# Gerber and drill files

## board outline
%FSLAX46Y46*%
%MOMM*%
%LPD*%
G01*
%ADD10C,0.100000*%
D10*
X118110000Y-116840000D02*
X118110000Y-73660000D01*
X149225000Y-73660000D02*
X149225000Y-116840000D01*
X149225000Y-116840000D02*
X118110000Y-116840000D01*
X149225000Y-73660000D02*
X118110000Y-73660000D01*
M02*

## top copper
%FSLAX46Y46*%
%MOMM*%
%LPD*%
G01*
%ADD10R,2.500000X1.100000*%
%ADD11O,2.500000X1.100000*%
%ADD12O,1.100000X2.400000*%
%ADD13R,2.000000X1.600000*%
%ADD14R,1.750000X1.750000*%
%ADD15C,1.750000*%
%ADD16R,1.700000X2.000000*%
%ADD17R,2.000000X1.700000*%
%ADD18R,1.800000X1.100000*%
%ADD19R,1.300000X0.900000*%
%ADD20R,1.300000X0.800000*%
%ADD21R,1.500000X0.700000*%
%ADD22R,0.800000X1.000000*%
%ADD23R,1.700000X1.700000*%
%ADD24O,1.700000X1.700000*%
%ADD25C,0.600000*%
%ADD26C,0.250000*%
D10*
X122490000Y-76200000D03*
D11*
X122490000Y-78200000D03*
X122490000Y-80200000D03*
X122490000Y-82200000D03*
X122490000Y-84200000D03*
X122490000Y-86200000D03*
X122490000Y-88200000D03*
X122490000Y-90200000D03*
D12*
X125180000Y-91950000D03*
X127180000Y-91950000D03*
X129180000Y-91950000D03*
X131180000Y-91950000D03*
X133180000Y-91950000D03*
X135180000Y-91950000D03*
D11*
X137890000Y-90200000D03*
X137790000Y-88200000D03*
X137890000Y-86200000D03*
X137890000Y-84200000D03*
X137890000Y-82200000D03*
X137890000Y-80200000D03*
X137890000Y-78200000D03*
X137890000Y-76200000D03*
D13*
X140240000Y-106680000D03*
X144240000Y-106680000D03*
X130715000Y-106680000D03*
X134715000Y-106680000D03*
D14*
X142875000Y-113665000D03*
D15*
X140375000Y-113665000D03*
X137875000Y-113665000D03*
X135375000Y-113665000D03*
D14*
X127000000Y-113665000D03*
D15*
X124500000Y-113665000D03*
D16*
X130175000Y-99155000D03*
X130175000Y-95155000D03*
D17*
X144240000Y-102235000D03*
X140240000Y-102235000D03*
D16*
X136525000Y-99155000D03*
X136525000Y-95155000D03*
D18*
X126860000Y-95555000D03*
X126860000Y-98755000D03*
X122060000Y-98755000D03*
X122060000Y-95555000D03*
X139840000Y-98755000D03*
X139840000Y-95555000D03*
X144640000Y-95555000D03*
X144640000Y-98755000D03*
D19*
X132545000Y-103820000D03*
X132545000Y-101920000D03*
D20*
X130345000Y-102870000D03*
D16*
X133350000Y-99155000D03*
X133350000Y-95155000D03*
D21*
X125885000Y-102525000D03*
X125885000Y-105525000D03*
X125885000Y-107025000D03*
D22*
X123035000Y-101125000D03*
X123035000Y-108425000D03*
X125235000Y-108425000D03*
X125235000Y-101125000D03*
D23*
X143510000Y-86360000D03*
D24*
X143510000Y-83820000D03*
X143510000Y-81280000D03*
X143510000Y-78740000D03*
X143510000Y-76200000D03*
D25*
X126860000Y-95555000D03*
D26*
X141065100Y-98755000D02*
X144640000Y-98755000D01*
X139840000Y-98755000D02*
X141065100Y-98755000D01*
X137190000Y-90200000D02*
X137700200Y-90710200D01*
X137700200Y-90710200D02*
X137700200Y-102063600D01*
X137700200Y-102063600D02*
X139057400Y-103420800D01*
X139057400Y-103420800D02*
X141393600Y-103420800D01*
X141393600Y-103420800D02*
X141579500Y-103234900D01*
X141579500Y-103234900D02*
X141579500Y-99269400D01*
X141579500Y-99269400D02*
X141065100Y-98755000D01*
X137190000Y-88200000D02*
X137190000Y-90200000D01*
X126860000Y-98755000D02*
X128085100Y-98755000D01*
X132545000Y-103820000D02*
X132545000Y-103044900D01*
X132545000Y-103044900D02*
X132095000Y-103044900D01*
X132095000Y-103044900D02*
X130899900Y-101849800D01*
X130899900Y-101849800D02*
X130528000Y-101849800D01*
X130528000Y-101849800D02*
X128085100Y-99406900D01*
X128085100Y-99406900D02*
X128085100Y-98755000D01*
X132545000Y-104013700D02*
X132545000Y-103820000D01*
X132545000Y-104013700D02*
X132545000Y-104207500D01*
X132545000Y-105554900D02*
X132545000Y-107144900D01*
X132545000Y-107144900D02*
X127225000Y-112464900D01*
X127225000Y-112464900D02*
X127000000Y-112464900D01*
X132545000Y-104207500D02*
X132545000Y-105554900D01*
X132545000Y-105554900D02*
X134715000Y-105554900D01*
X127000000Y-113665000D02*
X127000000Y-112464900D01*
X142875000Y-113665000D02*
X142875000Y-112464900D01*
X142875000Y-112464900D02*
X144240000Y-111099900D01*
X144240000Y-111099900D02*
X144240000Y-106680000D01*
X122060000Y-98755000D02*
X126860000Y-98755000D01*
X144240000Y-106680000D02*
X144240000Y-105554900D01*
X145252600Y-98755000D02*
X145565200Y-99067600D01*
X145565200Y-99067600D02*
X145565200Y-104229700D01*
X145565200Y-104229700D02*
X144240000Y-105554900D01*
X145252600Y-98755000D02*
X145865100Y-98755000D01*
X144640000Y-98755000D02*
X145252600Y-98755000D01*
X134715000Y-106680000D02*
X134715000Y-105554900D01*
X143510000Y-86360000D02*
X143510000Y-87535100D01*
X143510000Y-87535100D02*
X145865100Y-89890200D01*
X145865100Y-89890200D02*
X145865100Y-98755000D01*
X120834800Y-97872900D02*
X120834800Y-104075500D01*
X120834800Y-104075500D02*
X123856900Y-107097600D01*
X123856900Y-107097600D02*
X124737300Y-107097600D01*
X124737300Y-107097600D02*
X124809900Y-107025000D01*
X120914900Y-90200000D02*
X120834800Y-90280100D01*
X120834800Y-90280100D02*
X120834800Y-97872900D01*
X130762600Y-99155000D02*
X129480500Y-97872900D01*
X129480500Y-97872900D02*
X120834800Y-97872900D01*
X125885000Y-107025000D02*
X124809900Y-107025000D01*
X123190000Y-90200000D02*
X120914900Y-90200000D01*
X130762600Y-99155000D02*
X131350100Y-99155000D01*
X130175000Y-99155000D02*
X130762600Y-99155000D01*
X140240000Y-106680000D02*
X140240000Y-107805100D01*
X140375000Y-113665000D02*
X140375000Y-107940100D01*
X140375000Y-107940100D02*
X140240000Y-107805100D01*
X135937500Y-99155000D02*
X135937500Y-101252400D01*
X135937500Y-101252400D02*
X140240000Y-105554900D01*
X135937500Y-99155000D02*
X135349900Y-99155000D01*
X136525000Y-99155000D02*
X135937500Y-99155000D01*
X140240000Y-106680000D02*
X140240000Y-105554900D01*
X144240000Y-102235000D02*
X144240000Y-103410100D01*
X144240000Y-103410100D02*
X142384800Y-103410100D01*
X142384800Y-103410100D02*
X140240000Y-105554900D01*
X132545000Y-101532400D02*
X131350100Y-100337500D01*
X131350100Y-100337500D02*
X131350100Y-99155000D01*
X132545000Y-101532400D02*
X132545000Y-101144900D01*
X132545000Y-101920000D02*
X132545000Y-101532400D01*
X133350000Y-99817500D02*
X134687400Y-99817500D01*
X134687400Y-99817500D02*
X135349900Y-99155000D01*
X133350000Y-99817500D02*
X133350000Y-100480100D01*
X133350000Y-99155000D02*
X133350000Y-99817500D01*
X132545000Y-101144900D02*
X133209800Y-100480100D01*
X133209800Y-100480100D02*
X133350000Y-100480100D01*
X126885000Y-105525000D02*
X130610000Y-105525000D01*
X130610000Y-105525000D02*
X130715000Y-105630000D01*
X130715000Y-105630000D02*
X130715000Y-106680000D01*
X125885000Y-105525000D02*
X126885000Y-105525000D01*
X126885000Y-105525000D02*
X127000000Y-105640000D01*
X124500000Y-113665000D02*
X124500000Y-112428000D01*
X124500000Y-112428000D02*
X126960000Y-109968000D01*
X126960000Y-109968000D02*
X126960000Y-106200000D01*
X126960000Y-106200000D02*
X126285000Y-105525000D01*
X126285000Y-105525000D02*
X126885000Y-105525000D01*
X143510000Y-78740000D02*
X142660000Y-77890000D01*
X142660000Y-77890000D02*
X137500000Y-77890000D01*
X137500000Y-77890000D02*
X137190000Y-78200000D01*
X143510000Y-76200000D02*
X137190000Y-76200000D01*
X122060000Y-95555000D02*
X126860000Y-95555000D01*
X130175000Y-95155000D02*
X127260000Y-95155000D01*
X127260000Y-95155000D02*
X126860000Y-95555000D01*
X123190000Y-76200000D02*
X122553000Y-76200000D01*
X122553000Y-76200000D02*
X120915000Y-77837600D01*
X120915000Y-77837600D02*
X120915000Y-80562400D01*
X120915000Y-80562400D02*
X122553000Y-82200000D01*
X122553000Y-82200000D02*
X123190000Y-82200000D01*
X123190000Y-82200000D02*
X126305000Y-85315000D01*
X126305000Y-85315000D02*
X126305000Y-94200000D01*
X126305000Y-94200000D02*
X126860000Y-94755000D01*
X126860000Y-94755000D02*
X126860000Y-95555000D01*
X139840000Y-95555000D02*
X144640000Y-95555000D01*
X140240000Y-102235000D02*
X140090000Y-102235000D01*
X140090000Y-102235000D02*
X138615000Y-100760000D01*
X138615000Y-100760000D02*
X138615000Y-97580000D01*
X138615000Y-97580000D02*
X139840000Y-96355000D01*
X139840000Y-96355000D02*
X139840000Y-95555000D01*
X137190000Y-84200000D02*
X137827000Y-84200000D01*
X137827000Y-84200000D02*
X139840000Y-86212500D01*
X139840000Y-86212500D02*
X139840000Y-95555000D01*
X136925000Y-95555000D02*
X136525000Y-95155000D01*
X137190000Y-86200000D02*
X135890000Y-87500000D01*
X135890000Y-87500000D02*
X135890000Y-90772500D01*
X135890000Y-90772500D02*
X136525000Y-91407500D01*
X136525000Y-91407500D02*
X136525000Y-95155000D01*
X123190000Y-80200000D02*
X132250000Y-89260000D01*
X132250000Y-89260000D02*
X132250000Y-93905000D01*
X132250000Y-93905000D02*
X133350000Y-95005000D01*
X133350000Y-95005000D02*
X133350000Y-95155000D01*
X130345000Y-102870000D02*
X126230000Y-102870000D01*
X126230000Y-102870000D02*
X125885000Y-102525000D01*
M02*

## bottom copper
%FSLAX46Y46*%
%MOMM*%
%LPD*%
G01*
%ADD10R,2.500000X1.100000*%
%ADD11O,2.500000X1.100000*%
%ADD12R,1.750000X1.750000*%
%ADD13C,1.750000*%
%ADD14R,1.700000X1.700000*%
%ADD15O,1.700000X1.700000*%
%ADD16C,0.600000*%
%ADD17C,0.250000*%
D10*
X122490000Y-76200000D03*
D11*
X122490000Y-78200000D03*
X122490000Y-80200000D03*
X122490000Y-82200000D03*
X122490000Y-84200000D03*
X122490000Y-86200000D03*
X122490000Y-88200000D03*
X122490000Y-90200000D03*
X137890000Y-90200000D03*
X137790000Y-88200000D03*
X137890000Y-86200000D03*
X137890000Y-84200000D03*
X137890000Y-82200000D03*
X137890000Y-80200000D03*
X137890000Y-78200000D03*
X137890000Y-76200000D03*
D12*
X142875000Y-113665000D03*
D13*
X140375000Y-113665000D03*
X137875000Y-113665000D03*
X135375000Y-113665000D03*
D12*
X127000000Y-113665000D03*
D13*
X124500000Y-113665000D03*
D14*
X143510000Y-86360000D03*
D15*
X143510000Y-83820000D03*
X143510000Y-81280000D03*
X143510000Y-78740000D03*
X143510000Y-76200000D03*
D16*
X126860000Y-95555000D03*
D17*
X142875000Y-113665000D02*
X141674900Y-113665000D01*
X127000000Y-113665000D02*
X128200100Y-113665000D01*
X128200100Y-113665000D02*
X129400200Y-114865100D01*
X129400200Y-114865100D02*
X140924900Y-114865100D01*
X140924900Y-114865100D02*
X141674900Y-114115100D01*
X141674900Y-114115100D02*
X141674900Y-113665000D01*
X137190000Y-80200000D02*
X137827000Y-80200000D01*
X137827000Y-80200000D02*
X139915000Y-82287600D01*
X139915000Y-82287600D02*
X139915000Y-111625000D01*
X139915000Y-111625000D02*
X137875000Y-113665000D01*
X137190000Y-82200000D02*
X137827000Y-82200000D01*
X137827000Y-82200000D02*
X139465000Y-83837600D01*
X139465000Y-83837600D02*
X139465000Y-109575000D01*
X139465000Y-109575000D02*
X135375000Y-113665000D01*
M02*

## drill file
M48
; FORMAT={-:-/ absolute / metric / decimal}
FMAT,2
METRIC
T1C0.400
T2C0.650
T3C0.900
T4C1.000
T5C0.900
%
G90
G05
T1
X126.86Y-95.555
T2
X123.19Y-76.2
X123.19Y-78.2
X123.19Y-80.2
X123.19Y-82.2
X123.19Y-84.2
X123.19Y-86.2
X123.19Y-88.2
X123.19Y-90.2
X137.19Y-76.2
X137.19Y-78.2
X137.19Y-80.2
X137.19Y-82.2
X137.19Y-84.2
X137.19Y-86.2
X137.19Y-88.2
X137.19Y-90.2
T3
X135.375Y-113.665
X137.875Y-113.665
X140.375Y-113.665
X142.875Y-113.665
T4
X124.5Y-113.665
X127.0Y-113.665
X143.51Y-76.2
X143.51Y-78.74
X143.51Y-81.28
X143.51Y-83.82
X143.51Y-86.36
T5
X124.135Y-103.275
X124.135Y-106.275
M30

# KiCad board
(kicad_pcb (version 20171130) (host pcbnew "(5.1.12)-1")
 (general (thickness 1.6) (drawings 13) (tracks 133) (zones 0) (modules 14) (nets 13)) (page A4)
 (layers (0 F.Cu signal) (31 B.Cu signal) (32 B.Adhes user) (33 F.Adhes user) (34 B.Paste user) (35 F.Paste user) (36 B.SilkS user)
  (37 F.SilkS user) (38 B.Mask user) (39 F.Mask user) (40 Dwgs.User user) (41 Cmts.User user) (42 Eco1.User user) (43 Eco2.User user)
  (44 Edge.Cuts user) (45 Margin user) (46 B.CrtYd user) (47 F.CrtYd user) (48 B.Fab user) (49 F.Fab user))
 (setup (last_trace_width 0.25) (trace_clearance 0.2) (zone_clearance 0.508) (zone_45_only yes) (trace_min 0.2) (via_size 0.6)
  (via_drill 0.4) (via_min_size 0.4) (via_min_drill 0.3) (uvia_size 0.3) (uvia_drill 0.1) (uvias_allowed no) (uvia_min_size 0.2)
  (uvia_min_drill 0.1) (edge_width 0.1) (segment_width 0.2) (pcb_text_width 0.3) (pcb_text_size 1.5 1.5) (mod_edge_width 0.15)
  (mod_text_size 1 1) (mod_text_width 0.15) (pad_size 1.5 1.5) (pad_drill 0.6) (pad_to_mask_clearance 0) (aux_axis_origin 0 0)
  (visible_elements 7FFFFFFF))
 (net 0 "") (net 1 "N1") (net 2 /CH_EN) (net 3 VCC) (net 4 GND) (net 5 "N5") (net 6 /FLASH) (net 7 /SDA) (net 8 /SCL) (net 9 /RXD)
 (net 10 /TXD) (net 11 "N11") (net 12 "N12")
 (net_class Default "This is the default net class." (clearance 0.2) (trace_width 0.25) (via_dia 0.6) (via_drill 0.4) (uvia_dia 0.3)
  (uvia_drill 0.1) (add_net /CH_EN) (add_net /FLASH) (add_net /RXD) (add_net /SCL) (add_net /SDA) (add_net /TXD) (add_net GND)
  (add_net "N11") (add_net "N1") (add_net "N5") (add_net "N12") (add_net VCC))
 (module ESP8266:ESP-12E (layer F.Cu) (at 123.19 76.2)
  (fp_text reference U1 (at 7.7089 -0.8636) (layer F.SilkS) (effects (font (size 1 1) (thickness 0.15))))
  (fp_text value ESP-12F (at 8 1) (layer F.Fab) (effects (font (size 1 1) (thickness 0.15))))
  (pad 1 thru_hole rect (at 0 0) (size 2.5 1.1) (drill 0.65 (offset -0.7 0)) (layers *.Cu *.Mask F.SilkS) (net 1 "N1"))
  (pad 2 thru_hole oval (at 0 2) (size 2.5 1.1) (drill 0.65 (offset -0.7 0)) (layers *.Cu *.Mask F.SilkS))
  (pad 3 thru_hole oval (at 0 4) (size 2.5 1.1) (drill 0.65 (offset -0.7 0)) (layers *.Cu *.Mask F.SilkS) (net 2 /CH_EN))
  (pad 4 thru_hole oval (at 0 6) (size 2.5 1.1) (drill 0.65 (offset -0.7 0)) (layers *.Cu *.Mask F.SilkS) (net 1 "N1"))
  (pad 5 thru_hole oval (at 0 8) (size 2.5 1.1) (drill 0.65 (offset -0.7 0)) (layers *.Cu *.Mask F.SilkS))
  (pad 6 thru_hole oval (at 0 10) (size 2.5 1.1) (drill 0.65 (offset -0.7 0)) (layers *.Cu *.Mask F.SilkS))
  (pad 7 thru_hole oval (at 0 12) (size 2.5 1.1) (drill 0.65 (offset -0.7 0)) (layers *.Cu *.Mask F.SilkS))
  (pad 8 thru_hole oval (at 0 14) (size 2.5 1.1) (drill 0.65 (offset -0.7 0)) (layers *.Cu *.Mask F.SilkS) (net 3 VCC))
  (pad 9 smd oval (at 1.99 15.75 90) (size 2.4 1.1) (layers F.Cu F.Paste F.Mask))
  (pad 10 smd oval (at 3.99 15.75 90) (size 2.4 1.1) (layers F.Cu F.Paste F.Mask))
  (pad 11 smd oval (at 5.99 15.75 90) (size 2.4 1.1) (layers F.Cu F.Paste F.Mask))
  (pad 12 smd oval (at 7.99 15.75 90) (size 2.4 1.1) (layers F.Cu F.Paste F.Mask))
  (pad 13 smd oval (at 9.99 15.75 90) (size 2.4 1.1) (layers F.Cu F.Paste F.Mask))
  (pad 14 smd oval (at 11.99 15.75 90) (size 2.4 1.1) (layers F.Cu F.Paste F.Mask))
  (pad 15 thru_hole oval (at 14 14) (size 2.5 1.1) (drill 0.65 (offset 0.7 0)) (layers *.Cu *.Mask F.SilkS) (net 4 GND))
  (pad 16 thru_hole oval (at 14 12) (size 2.5 1.1) (drill 0.65 (offset 0.6 0)) (layers *.Cu *.Mask F.SilkS) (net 4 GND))
  (pad 17 thru_hole oval (at 14 10) (size 2.5 1.1) (drill 0.65 (offset 0.7 0)) (layers *.Cu *.Mask F.SilkS) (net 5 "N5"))
  (pad 18 thru_hole oval (at 14 8) (size 2.5 1.1) (drill 0.65 (offset 0.7 0)) (layers *.Cu *.Mask F.SilkS) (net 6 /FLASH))
  (pad 19 thru_hole oval (at 14 6) (size 2.5 1.1) (drill 0.65 (offset 0.7 0)) (layers *.Cu *.Mask F.SilkS) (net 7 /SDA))
  (pad 20 thru_hole oval (at 14 4) (size 2.5 1.1) (drill 0.65 (offset 0.7 0)) (layers *.Cu *.Mask F.SilkS) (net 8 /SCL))
  (pad 21 thru_hole oval (at 14 2) (size 2.5 1.1) (drill 0.65 (offset 0.7 0)) (layers *.Cu *.Mask F.SilkS) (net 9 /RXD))
  (pad 22 thru_hole oval (at 14 0) (size 2.5 1.1) (drill 0.65 (offset 0.7 0)) (layers *.Cu *.Mask F.SilkS) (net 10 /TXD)))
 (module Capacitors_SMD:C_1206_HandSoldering (layer F.Cu) (at 142.24 106.68)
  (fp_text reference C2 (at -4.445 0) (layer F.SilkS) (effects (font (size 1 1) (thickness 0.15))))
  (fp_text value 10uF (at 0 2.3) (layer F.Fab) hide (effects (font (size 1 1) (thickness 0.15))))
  (pad 1 smd rect (at -2 0) (size 2 1.6) (layers F.Cu F.Paste F.Mask) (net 3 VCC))
  (pad 2 smd rect (at 2 0) (size 2 1.6) (layers F.Cu F.Paste F.Mask) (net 4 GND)))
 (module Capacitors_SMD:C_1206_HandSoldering (layer F.Cu) (at 132.715 106.68)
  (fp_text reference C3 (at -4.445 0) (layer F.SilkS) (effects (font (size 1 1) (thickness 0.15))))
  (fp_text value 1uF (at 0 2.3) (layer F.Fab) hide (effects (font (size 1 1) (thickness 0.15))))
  (pad 1 smd rect (at -2 0) (size 2 1.6) (layers F.Cu F.Paste F.Mask) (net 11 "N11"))
  (pad 2 smd rect (at 2 0) (size 2 1.6) (layers F.Cu F.Paste F.Mask) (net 4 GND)))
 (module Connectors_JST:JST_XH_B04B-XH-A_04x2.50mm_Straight (layer F.Cu) (at 142.875 113.665 180)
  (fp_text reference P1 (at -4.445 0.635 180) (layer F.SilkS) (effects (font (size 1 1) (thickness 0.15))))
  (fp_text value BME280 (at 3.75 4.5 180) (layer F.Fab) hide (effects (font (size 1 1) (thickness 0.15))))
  (pad 1 thru_hole rect (at 0 0 180) (size 1.75 1.75) (drill 0.9) (layers *.Cu *.Mask) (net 4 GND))
  (pad 2 thru_hole circle (at 2.5 0 180) (size 1.75 1.75) (drill 0.9) (layers *.Cu *.Mask) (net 3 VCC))
  (pad 3 thru_hole circle (at 5 0 180) (size 1.75 1.75) (drill 0.9) (layers *.Cu *.Mask) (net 8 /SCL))
  (pad 4 thru_hole circle (at 7.5 0 180) (size 1.75 1.75) (drill 0.9) (layers *.Cu *.Mask) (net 7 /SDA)))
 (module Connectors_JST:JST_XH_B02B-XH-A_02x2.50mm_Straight (layer F.Cu) (at 127 113.665 180)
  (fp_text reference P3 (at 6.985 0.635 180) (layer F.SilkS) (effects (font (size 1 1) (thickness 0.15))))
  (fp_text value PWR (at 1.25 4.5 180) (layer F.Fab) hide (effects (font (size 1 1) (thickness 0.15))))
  (pad 1 thru_hole rect (at 0 0 180) (size 1.75 1.75) (drill 1) (layers *.Cu *.Mask) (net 4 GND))
  (pad 2 thru_hole circle (at 2.5 0 180) (size 1.75 1.75) (drill 1) (layers *.Cu *.Mask) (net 11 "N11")))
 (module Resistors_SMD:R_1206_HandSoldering (layer F.Cu) (at 130.175 97.155 90)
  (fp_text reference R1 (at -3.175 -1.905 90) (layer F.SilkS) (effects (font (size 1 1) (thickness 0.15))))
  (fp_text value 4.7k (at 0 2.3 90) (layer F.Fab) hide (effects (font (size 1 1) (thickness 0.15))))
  (pad 1 smd rect (at -2 0 90) (size 2 1.7) (layers F.Cu F.Paste F.Mask) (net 3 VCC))
  (pad 2 smd rect (at 2 0 90) (size 2 1.7) (layers F.Cu F.Paste F.Mask) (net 1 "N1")))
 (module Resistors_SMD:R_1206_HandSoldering (layer F.Cu) (at 142.24 102.235 180)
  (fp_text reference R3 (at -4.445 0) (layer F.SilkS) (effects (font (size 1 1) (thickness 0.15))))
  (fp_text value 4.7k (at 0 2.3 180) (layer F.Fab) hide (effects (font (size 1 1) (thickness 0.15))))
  (pad 1 smd rect (at -2 0 180) (size 2 1.7) (layers F.Cu F.Paste F.Mask) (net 3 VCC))
  (pad 2 smd rect (at 2 0 180) (size 2 1.7) (layers F.Cu F.Paste F.Mask) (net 6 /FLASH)))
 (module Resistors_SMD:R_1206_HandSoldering (layer F.Cu) (at 136.525 97.155 90)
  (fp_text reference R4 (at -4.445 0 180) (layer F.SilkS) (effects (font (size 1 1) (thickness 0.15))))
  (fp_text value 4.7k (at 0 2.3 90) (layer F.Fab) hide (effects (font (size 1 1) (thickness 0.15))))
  (pad 1 smd rect (at -2 0 90) (size 2 1.7) (layers F.Cu F.Paste F.Mask) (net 3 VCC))
  (pad 2 smd rect (at 2 0 90) (size 2 1.7) (layers F.Cu F.Paste F.Mask) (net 5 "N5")))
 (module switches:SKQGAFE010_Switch (layer F.Cu) (at 124.46 97.155 180)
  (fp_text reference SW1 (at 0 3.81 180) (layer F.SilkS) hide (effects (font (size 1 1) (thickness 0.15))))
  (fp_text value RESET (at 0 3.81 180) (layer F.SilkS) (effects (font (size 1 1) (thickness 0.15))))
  (pad 3 smd rect (at -2.4 1.6 180) (size 1.8 1.1) (layers F.Cu F.Paste F.Mask) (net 1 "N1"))
  (pad 1 smd rect (at -2.4 -1.6 180) (size 1.8 1.1) (layers F.Cu F.Paste F.Mask) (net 4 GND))
  (pad 2 smd rect (at 2.4 -1.6 180) (size 1.8 1.1) (layers F.Cu F.Paste F.Mask) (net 4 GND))
  (pad 4 smd rect (at 2.4 1.6 180) (size 1.8 1.1) (layers F.Cu F.Paste F.Mask) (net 1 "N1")))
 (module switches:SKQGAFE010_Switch (layer F.Cu) (at 142.24 97.155)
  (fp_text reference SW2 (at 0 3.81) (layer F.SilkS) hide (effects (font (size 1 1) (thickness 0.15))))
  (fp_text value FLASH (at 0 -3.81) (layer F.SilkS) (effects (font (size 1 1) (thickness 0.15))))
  (pad 3 smd rect (at -2.4 1.6) (size 1.8 1.1) (layers F.Cu F.Paste F.Mask) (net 4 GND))
  (pad 1 smd rect (at -2.4 -1.6) (size 1.8 1.1) (layers F.Cu F.Paste F.Mask) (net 6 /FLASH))
  (pad 2 smd rect (at 2.4 -1.6) (size 1.8 1.1) (layers F.Cu F.Paste F.Mask) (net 6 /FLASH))
  (pad 4 smd rect (at 2.4 1.6) (size 1.8 1.1) (layers F.Cu F.Paste F.Mask) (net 4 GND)))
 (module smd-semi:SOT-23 (layer F.Cu) (at 131.445 102.87 180)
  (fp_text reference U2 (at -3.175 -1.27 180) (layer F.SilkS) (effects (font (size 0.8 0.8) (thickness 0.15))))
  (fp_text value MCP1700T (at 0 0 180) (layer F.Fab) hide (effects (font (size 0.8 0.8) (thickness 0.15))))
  (pad 1 smd rect (at -1.1 -0.95 180) (size 1.3 0.9) (layers F.Cu F.Paste F.Mask) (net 4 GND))
  (pad 2 smd rect (at -1.1 0.95 180) (size 1.3 0.9) (layers F.Cu F.Paste F.Mask) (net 3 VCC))
  (pad 3 smd rect (at 1.1 0 180) (size 1.3 0.8) (layers F.Cu F.Paste F.Mask) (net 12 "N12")))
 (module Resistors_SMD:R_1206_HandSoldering (layer F.Cu) (at 133.35 97.155 90)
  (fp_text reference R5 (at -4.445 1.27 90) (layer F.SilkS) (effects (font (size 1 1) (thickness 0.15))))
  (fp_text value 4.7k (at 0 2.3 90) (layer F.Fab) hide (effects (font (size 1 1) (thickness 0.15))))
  (pad 1 smd rect (at -2 0 90) (size 2 1.7) (layers F.Cu F.Paste F.Mask) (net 3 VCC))
  (pad 2 smd rect (at 2 0 90) (size 2 1.7) (layers F.Cu F.Paste F.Mask) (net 2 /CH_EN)))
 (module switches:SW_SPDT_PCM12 (layer F.Cu) (at 124.46 104.775 270)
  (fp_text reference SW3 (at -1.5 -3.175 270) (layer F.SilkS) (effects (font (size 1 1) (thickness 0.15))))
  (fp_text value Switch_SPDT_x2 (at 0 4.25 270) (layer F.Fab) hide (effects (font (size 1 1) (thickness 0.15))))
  (pad "" np_thru_hole circle (at -1.5 0.325 270) (size 0.9 0.9) (drill 0.9) (layers *.Cu *.Mask))
  (pad "" np_thru_hole circle (at 1.5 0.325 270) (size 0.9 0.9) (drill 0.9) (layers *.Cu *.Mask))
  (pad 1 smd rect (at -2.25 -1.425 270) (size 0.7 1.5) (layers F.Cu F.Paste F.Mask) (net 12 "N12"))
  (pad 2 smd rect (at 0.75 -1.425 270) (size 0.7 1.5) (layers F.Cu F.Paste F.Mask) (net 11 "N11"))
  (pad 3 smd rect (at 2.25 -1.425 270) (size 0.7 1.5) (layers F.Cu F.Paste F.Mask) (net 3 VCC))
  (pad "" smd rect (at -3.65 1.425 270) (size 1 0.8) (layers F.Cu F.Paste F.Mask))
  (pad "" smd rect (at 3.65 1.425 270) (size 1 0.8) (layers F.Cu F.Paste F.Mask))
  (pad "" smd rect (at 3.65 -0.775 270) (size 1 0.8) (layers F.Cu F.Paste F.Mask))
  (pad "" smd rect (at -3.65 -0.775 270) (size 1 0.8) (layers F.Cu F.Paste F.Mask)))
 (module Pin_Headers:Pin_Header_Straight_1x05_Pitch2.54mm (layer F.Cu) (at 143.51 86.36 180)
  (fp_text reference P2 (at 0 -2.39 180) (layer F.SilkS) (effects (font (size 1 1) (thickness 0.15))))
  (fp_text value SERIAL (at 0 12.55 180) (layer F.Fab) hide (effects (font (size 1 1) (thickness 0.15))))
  (pad 1 thru_hole rect (at 0 0 180) (size 1.7 1.7) (drill 1) (layers *.Cu *.Mask) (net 4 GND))
  (pad 2 thru_hole oval (at 0 2.54 180) (size 1.7 1.7) (drill 1) (layers *.Cu *.Mask))
  (pad 3 thru_hole oval (at 0 5.08 180) (size 1.7 1.7) (drill 1) (layers *.Cu *.Mask))
  (pad 4 thru_hole oval (at 0 7.62 180) (size 1.7 1.7) (drill 1) (layers *.Cu *.Mask) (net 9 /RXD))
  (pad 5 thru_hole oval (at 0 10.16 180) (size 1.7 1.7) (drill 1) (layers *.Cu *.Mask) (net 10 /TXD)))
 (gr_line (start 118.11 116.84) (end 118.11 73.66) (layer Edge.Cuts) (width 0.1))
 (gr_line (start 149.225 73.66) (end 149.225 116.84) (layer Edge.Cuts) (width 0.1))
 (gr_line (start 149.225 116.84) (end 118.11 116.84) (layer Edge.Cuts) (width 0.1))
 (gr_line (start 149.225 73.66) (end 118.11 73.66) (layer Edge.Cuts) (width 0.1))
 (segment (start 141.0651 98.755) (end 144.64 98.755) (width 0.25) (layer F.Cu) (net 4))
 (segment (start 139.84 98.755) (end 141.0651 98.755) (width 0.25) (layer F.Cu) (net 4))
 (segment (start 137.19 90.2) (end 137.7002 90.7102) (width 0.25) (layer F.Cu) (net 4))
 (segment (start 137.7002 90.7102) (end 137.7002 102.0636) (width 0.25) (layer F.Cu) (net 4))
 (segment (start 137.7002 102.0636) (end 139.0574 103.4208) (width 0.25) (layer F.Cu) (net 4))
 (segment (start 139.0574 103.4208) (end 141.3936 103.4208) (width 0.25) (layer F.Cu) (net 4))
 (segment (start 141.3936 103.4208) (end 141.5795 103.2349) (width 0.25) (layer F.Cu) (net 4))
 (segment (start 141.5795 103.2349) (end 141.5795 99.2694) (width 0.25) (layer F.Cu) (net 4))
 (segment (start 141.5795 99.2694) (end 141.0651 98.755) (width 0.25) (layer F.Cu) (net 4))
 (segment (start 137.19 88.2) (end 137.19 90.2) (width 0.25) (layer F.Cu) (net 4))
 (segment (start 126.86 98.755) (end 128.0851 98.755) (width 0.25) (layer F.Cu) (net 4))
 (segment (start 132.545 103.82) (end 132.545 103.0449) (width 0.25) (layer F.Cu) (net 4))
 (segment (start 132.545 103.0449) (end 132.095 103.0449) (width 0.25) (layer F.Cu) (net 4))
 (segment (start 132.095 103.0449) (end 130.8999 101.8498) (width 0.25) (layer F.Cu) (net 4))
 (segment (start 130.8999 101.8498) (end 130.528 101.8498) (width 0.25) (layer F.Cu) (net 4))
 (segment (start 130.528 101.8498) (end 128.0851 99.4069) (width 0.25) (layer F.Cu) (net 4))
 (segment (start 128.0851 99.4069) (end 128.0851 98.755) (width 0.25) (layer F.Cu) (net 4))
 (segment (start 132.545 104.0137) (end 132.545 103.82) (width 0.25) (layer F.Cu) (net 4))
 (segment (start 132.545 104.0137) (end 132.545 104.2075) (width 0.25) (layer F.Cu) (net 4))
 (segment (start 132.545 105.5549) (end 132.545 107.1449) (width 0.25) (layer F.Cu) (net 4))
 (segment (start 132.545 107.1449) (end 127.225 112.4649) (width 0.25) (layer F.Cu) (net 4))
 (segment (start 127.225 112.4649) (end 127 112.4649) (width 0.25) (layer F.Cu) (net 4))
 (segment (start 132.545 104.2075) (end 132.545 105.5549) (width 0.25) (layer F.Cu) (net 4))
 (segment (start 132.545 105.5549) (end 134.715 105.5549) (width 0.25) (layer F.Cu) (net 4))
 (segment (start 127 113.665) (end 127 112.4649) (width 0.25) (layer F.Cu) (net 4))
 (segment (start 142.875 113.665) (end 142.875 112.4649) (width 0.25) (layer F.Cu) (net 4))
 (segment (start 142.875 112.4649) (end 144.24 111.0999) (width 0.25) (layer F.Cu) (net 4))
 (segment (start 144.24 111.0999) (end 144.24 106.68) (width 0.25) (layer F.Cu) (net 4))
 (segment (start 142.875 113.665) (end 141.6749 113.665) (width 0.25) (layer B.Cu) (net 4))
 (segment (start 127 113.665) (end 128.2001 113.665) (width 0.25) (layer B.Cu) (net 4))
 (segment (start 128.2001 113.665) (end 129.4002 114.8651) (width 0.25) (layer B.Cu) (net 4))
 (segment (start 129.4002 114.8651) (end 140.9249 114.8651) (width 0.25) (layer B.Cu) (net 4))
 (segment (start 140.9249 114.8651) (end 141.6749 114.1151) (width 0.25) (layer B.Cu) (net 4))
 (segment (start 141.6749 114.1151) (end 141.6749 113.665) (width 0.25) (layer B.Cu) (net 4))
 (segment (start 122.06 98.755) (end 126.86 98.755) (width 0.25) (layer F.Cu) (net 4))
 (segment (start 144.24 106.68) (end 144.24 105.5549) (width 0.25) (layer F.Cu) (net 4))
 (segment (start 145.2526 98.755) (end 145.5652 99.0676) (width 0.25) (layer F.Cu) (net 4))
 (segment (start 145.5652 99.0676) (end 145.5652 104.2297) (width 0.25) (layer F.Cu) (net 4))
 (segment (start 145.5652 104.2297) (end 144.24 105.5549) (width 0.25) (layer F.Cu) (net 4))
 (segment (start 145.2526 98.755) (end 145.8651 98.755) (width 0.25) (layer F.Cu) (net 4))
 (segment (start 144.64 98.755) (end 145.2526 98.755) (width 0.25) (layer F.Cu) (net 4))
 (segment (start 134.715 106.68) (end 134.715 105.5549) (width 0.25) (layer F.Cu) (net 4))
 (segment (start 143.51 86.36) (end 143.51 87.5351) (width 0.25) (layer F.Cu) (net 4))
 (segment (start 143.51 87.5351) (end 145.8651 89.8902) (width 0.25) (layer F.Cu) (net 4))
 (segment (start 145.8651 89.8902) (end 145.8651 98.755) (width 0.25) (layer F.Cu) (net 4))
 (segment (start 120.8348 97.8729) (end 120.8348 104.0755) (width 0.25) (layer F.Cu) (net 3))
 (segment (start 120.8348 104.0755) (end 123.8569 107.0976) (width 0.25) (layer F.Cu) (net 3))
 (segment (start 123.8569 107.0976) (end 124.7373 107.0976) (width 0.25) (layer F.Cu) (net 3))
 (segment (start 124.7373 107.0976) (end 124.8099 107.025) (width 0.25) (layer F.Cu) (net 3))
 (segment (start 120.9149 90.2) (end 120.8348 90.2801) (width 0.25) (layer F.Cu) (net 3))
 (segment (start 120.8348 90.2801) (end 120.8348 97.8729) (width 0.25) (layer F.Cu) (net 3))
 (segment (start 130.7626 99.155) (end 129.4805 97.8729) (width 0.25) (layer F.Cu) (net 3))
 (segment (start 129.4805 97.8729) (end 120.8348 97.8729) (width 0.25) (layer F.Cu) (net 3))
 (segment (start 125.885 107.025) (end 124.8099 107.025) (width 0.25) (layer F.Cu) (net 3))
 (segment (start 123.19 90.2) (end 120.9149 90.2) (width 0.25) (layer F.Cu) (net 3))
 (segment (start 130.7626 99.155) (end 131.3501 99.155) (width 0.25) (layer F.Cu) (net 3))
 (segment (start 130.175 99.155) (end 130.7626 99.155) (width 0.25) (layer F.Cu) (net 3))
 (segment (start 140.24 106.68) (end 140.24 107.8051) (width 0.25) (layer F.Cu) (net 3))
 (segment (start 140.375 113.665) (end 140.375 107.9401) (width 0.25) (layer F.Cu) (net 3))
 (segment (start 140.375 107.9401) (end 140.24 107.8051) (width 0.25) (layer F.Cu) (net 3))
 (segment (start 135.9375 99.155) (end 135.9375 101.2524) (width 0.25) (layer F.Cu) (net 3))
 (segment (start 135.9375 101.2524) (end 140.24 105.5549) (width 0.25) (layer F.Cu) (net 3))
 (segment (start 135.9375 99.155) (end 135.3499 99.155) (width 0.25) (layer F.Cu) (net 3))
 (segment (start 136.525 99.155) (end 135.9375 99.155) (width 0.25) (layer F.Cu) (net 3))
 (segment (start 140.24 106.68) (end 140.24 105.5549) (width 0.25) (layer F.Cu) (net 3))
 (segment (start 144.24 102.235) (end 144.24 103.4101) (width 0.25) (layer F.Cu) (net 3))
 (segment (start 144.24 103.4101) (end 142.3848 103.4101) (width 0.25) (layer F.Cu) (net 3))
 (segment (start 142.3848 103.4101) (end 140.24 105.5549) (width 0.25) (layer F.Cu) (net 3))
 (segment (start 132.545 101.5324) (end 131.3501 100.3375) (width 0.25) (layer F.Cu) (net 3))
 (segment (start 131.3501 100.3375) (end 131.3501 99.155) (width 0.25) (layer F.Cu) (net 3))
 (segment (start 132.545 101.5324) (end 132.545 101.1449) (width 0.25) (layer F.Cu) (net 3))
 (segment (start 132.545 101.92) (end 132.545 101.5324) (width 0.25) (layer F.Cu) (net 3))
 (segment (start 133.35 99.8175) (end 134.6874 99.8175) (width 0.25) (layer F.Cu) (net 3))
 (segment (start 134.6874 99.8175) (end 135.3499 99.155) (width 0.25) (layer F.Cu) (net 3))
 (segment (start 133.35 99.8175) (end 133.35 100.4801) (width 0.25) (layer F.Cu) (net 3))
 (segment (start 133.35 99.155) (end 133.35 99.8175) (width 0.25) (layer F.Cu) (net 3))
 (segment (start 132.545 101.1449) (end 133.2098 100.4801) (width 0.25) (layer F.Cu) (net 3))
 (segment (start 133.2098 100.4801) (end 133.35 100.4801) (width 0.25) (layer F.Cu) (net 3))
 (segment (start 126.885 105.525) (end 130.61 105.525) (width 0.25) (layer F.Cu) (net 11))
 (segment (start 130.61 105.525) (end 130.715 105.63) (width 0.25) (layer F.Cu) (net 11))
 (segment (start 130.715 105.63) (end 130.715 106.68) (width 0.25) (layer F.Cu) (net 11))
 (segment (start 125.885 105.525) (end 126.885 105.525) (width 0.25) (layer F.Cu) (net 11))
 (segment (start 126.885 105.525) (end 127 105.64) (width 0.25) (layer F.Cu) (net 11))
 (segment (start 124.5 113.665) (end 124.5 112.428) (width 0.25) (layer F.Cu) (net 11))
 (segment (start 124.5 112.428) (end 126.96 109.968) (width 0.25) (layer F.Cu) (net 11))
 (segment (start 126.96 109.968) (end 126.96 106.2) (width 0.25) (layer F.Cu) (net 11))
 (segment (start 126.96 106.2) (end 126.285 105.525) (width 0.25) (layer F.Cu) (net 11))
 (segment (start 126.285 105.525) (end 126.885 105.525) (width 0.25) (layer F.Cu) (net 11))
 (segment (start 137.19 80.2) (end 137.827 80.2) (width 0.25) (layer B.Cu) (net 8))
 (segment (start 137.827 80.2) (end 139.915 82.2876) (width 0.25) (layer B.Cu) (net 8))
 (segment (start 139.915 82.2876) (end 139.915 111.625) (width 0.25) (layer B.Cu) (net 8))
 (segment (start 139.915 111.625) (end 137.875 113.665) (width 0.25) (layer B.Cu) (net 8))
 (segment (start 137.19 82.2) (end 137.827 82.2) (width 0.25) (layer B.Cu) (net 7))
 (segment (start 137.827 82.2) (end 139.465 83.8376) (width 0.25) (layer B.Cu) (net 7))
 (segment (start 139.465 83.8376) (end 139.465 109.575) (width 0.25) (layer B.Cu) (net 7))
 (segment (start 139.465 109.575) (end 135.375 113.665) (width 0.25) (layer B.Cu) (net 7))
 (segment (start 143.51 78.74) (end 142.66 77.89) (width 0.25) (layer F.Cu) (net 9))
 (segment (start 142.66 77.89) (end 137.5 77.89) (width 0.25) (layer F.Cu) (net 9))
 (segment (start 137.5 77.89) (end 137.19 78.2) (width 0.25) (layer F.Cu) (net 9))
 (segment (start 143.51 76.2) (end 137.19 76.2) (width 0.25) (layer F.Cu) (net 10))
 (segment (start 122.06 95.555) (end 126.86 95.555) (width 0.25) (layer F.Cu) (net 1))
 (segment (start 130.175 95.155) (end 127.26 95.155) (width 0.25) (layer F.Cu) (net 1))
 (segment (start 127.26 95.155) (end 126.86 95.555) (width 0.25) (layer F.Cu) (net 1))
 (segment (start 123.19 76.2) (end 122.553 76.2) (width 0.25) (layer F.Cu) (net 1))
 (segment (start 122.553 76.2) (end 120.915 77.8376) (width 0.25) (layer F.Cu) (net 1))
 (segment (start 120.915 77.8376) (end 120.915 80.5624) (width 0.25) (layer F.Cu) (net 1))
 (segment (start 120.915 80.5624) (end 122.553 82.2) (width 0.25) (layer F.Cu) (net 1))
 (segment (start 122.553 82.2) (end 123.19 82.2) (width 0.25) (layer F.Cu) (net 1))
 (segment (start 123.19 82.2) (end 126.305 85.315) (width 0.25) (layer F.Cu) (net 1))
 (segment (start 126.305 85.315) (end 126.305 94.2) (width 0.25) (layer F.Cu) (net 1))
 (segment (start 126.305 94.2) (end 126.86 94.755) (width 0.25) (layer F.Cu) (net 1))
 (segment (start 126.86 94.755) (end 126.86 95.555) (width 0.25) (layer F.Cu) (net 1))
 (via (at 126.86 95.555) (size 0.6) (layers F.Cu B.Cu) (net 1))
 (segment (start 139.84 95.555) (end 144.64 95.555) (width 0.25) (layer F.Cu) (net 6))
 (segment (start 140.24 102.235) (end 140.09 102.235) (width 0.25) (layer F.Cu) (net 6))
 (segment (start 140.09 102.235) (end 138.615 100.76) (width 0.25) (layer F.Cu) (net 6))
 (segment (start 138.615 100.76) (end 138.615 97.58) (width 0.25) (layer F.Cu) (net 6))
 (segment (start 138.615 97.58) (end 139.84 96.355) (width 0.25) (layer F.Cu) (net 6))
 (segment (start 139.84 96.355) (end 139.84 95.555) (width 0.25) (layer F.Cu) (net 6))
 (segment (start 137.19 84.2) (end 137.827 84.2) (width 0.25) (layer F.Cu) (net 6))
 (segment (start 137.827 84.2) (end 139.84 86.2125) (width 0.25) (layer F.Cu) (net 6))
 (segment (start 139.84 86.2125) (end 139.84 95.555) (width 0.25) (layer F.Cu) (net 6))
 (segment (start 136.925 95.555) (end 136.525 95.155) (width 0.25) (layer F.Cu) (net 5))
 (segment (start 137.19 86.2) (end 135.89 87.5) (width 0.25) (layer F.Cu) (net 5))
 (segment (start 135.89 87.5) (end 135.89 90.7725) (width 0.25) (layer F.Cu) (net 5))
 (segment (start 135.89 90.7725) (end 136.525 91.4075) (width 0.25) (layer F.Cu) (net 5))
 (segment (start 136.525 91.4075) (end 136.525 95.155) (width 0.25) (layer F.Cu) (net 5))
 (segment (start 123.19 80.2) (end 132.25 89.26) (width 0.25) (layer F.Cu) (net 2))
 (segment (start 132.25 89.26) (end 132.25 93.905) (width 0.25) (layer F.Cu) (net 2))
 (segment (start 132.25 93.905) (end 133.35 95.005) (width 0.25) (layer F.Cu) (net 2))
 (segment (start 133.35 95.005) (end 133.35 95.155) (width 0.25) (layer F.Cu) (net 2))
 (segment (start 130.345 102.87) (end 126.23 102.87) (width 0.25) (layer F.Cu) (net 12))
 (segment (start 126.23 102.87) (end 125.885 102.525) (width 0.25) (layer F.Cu) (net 12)))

